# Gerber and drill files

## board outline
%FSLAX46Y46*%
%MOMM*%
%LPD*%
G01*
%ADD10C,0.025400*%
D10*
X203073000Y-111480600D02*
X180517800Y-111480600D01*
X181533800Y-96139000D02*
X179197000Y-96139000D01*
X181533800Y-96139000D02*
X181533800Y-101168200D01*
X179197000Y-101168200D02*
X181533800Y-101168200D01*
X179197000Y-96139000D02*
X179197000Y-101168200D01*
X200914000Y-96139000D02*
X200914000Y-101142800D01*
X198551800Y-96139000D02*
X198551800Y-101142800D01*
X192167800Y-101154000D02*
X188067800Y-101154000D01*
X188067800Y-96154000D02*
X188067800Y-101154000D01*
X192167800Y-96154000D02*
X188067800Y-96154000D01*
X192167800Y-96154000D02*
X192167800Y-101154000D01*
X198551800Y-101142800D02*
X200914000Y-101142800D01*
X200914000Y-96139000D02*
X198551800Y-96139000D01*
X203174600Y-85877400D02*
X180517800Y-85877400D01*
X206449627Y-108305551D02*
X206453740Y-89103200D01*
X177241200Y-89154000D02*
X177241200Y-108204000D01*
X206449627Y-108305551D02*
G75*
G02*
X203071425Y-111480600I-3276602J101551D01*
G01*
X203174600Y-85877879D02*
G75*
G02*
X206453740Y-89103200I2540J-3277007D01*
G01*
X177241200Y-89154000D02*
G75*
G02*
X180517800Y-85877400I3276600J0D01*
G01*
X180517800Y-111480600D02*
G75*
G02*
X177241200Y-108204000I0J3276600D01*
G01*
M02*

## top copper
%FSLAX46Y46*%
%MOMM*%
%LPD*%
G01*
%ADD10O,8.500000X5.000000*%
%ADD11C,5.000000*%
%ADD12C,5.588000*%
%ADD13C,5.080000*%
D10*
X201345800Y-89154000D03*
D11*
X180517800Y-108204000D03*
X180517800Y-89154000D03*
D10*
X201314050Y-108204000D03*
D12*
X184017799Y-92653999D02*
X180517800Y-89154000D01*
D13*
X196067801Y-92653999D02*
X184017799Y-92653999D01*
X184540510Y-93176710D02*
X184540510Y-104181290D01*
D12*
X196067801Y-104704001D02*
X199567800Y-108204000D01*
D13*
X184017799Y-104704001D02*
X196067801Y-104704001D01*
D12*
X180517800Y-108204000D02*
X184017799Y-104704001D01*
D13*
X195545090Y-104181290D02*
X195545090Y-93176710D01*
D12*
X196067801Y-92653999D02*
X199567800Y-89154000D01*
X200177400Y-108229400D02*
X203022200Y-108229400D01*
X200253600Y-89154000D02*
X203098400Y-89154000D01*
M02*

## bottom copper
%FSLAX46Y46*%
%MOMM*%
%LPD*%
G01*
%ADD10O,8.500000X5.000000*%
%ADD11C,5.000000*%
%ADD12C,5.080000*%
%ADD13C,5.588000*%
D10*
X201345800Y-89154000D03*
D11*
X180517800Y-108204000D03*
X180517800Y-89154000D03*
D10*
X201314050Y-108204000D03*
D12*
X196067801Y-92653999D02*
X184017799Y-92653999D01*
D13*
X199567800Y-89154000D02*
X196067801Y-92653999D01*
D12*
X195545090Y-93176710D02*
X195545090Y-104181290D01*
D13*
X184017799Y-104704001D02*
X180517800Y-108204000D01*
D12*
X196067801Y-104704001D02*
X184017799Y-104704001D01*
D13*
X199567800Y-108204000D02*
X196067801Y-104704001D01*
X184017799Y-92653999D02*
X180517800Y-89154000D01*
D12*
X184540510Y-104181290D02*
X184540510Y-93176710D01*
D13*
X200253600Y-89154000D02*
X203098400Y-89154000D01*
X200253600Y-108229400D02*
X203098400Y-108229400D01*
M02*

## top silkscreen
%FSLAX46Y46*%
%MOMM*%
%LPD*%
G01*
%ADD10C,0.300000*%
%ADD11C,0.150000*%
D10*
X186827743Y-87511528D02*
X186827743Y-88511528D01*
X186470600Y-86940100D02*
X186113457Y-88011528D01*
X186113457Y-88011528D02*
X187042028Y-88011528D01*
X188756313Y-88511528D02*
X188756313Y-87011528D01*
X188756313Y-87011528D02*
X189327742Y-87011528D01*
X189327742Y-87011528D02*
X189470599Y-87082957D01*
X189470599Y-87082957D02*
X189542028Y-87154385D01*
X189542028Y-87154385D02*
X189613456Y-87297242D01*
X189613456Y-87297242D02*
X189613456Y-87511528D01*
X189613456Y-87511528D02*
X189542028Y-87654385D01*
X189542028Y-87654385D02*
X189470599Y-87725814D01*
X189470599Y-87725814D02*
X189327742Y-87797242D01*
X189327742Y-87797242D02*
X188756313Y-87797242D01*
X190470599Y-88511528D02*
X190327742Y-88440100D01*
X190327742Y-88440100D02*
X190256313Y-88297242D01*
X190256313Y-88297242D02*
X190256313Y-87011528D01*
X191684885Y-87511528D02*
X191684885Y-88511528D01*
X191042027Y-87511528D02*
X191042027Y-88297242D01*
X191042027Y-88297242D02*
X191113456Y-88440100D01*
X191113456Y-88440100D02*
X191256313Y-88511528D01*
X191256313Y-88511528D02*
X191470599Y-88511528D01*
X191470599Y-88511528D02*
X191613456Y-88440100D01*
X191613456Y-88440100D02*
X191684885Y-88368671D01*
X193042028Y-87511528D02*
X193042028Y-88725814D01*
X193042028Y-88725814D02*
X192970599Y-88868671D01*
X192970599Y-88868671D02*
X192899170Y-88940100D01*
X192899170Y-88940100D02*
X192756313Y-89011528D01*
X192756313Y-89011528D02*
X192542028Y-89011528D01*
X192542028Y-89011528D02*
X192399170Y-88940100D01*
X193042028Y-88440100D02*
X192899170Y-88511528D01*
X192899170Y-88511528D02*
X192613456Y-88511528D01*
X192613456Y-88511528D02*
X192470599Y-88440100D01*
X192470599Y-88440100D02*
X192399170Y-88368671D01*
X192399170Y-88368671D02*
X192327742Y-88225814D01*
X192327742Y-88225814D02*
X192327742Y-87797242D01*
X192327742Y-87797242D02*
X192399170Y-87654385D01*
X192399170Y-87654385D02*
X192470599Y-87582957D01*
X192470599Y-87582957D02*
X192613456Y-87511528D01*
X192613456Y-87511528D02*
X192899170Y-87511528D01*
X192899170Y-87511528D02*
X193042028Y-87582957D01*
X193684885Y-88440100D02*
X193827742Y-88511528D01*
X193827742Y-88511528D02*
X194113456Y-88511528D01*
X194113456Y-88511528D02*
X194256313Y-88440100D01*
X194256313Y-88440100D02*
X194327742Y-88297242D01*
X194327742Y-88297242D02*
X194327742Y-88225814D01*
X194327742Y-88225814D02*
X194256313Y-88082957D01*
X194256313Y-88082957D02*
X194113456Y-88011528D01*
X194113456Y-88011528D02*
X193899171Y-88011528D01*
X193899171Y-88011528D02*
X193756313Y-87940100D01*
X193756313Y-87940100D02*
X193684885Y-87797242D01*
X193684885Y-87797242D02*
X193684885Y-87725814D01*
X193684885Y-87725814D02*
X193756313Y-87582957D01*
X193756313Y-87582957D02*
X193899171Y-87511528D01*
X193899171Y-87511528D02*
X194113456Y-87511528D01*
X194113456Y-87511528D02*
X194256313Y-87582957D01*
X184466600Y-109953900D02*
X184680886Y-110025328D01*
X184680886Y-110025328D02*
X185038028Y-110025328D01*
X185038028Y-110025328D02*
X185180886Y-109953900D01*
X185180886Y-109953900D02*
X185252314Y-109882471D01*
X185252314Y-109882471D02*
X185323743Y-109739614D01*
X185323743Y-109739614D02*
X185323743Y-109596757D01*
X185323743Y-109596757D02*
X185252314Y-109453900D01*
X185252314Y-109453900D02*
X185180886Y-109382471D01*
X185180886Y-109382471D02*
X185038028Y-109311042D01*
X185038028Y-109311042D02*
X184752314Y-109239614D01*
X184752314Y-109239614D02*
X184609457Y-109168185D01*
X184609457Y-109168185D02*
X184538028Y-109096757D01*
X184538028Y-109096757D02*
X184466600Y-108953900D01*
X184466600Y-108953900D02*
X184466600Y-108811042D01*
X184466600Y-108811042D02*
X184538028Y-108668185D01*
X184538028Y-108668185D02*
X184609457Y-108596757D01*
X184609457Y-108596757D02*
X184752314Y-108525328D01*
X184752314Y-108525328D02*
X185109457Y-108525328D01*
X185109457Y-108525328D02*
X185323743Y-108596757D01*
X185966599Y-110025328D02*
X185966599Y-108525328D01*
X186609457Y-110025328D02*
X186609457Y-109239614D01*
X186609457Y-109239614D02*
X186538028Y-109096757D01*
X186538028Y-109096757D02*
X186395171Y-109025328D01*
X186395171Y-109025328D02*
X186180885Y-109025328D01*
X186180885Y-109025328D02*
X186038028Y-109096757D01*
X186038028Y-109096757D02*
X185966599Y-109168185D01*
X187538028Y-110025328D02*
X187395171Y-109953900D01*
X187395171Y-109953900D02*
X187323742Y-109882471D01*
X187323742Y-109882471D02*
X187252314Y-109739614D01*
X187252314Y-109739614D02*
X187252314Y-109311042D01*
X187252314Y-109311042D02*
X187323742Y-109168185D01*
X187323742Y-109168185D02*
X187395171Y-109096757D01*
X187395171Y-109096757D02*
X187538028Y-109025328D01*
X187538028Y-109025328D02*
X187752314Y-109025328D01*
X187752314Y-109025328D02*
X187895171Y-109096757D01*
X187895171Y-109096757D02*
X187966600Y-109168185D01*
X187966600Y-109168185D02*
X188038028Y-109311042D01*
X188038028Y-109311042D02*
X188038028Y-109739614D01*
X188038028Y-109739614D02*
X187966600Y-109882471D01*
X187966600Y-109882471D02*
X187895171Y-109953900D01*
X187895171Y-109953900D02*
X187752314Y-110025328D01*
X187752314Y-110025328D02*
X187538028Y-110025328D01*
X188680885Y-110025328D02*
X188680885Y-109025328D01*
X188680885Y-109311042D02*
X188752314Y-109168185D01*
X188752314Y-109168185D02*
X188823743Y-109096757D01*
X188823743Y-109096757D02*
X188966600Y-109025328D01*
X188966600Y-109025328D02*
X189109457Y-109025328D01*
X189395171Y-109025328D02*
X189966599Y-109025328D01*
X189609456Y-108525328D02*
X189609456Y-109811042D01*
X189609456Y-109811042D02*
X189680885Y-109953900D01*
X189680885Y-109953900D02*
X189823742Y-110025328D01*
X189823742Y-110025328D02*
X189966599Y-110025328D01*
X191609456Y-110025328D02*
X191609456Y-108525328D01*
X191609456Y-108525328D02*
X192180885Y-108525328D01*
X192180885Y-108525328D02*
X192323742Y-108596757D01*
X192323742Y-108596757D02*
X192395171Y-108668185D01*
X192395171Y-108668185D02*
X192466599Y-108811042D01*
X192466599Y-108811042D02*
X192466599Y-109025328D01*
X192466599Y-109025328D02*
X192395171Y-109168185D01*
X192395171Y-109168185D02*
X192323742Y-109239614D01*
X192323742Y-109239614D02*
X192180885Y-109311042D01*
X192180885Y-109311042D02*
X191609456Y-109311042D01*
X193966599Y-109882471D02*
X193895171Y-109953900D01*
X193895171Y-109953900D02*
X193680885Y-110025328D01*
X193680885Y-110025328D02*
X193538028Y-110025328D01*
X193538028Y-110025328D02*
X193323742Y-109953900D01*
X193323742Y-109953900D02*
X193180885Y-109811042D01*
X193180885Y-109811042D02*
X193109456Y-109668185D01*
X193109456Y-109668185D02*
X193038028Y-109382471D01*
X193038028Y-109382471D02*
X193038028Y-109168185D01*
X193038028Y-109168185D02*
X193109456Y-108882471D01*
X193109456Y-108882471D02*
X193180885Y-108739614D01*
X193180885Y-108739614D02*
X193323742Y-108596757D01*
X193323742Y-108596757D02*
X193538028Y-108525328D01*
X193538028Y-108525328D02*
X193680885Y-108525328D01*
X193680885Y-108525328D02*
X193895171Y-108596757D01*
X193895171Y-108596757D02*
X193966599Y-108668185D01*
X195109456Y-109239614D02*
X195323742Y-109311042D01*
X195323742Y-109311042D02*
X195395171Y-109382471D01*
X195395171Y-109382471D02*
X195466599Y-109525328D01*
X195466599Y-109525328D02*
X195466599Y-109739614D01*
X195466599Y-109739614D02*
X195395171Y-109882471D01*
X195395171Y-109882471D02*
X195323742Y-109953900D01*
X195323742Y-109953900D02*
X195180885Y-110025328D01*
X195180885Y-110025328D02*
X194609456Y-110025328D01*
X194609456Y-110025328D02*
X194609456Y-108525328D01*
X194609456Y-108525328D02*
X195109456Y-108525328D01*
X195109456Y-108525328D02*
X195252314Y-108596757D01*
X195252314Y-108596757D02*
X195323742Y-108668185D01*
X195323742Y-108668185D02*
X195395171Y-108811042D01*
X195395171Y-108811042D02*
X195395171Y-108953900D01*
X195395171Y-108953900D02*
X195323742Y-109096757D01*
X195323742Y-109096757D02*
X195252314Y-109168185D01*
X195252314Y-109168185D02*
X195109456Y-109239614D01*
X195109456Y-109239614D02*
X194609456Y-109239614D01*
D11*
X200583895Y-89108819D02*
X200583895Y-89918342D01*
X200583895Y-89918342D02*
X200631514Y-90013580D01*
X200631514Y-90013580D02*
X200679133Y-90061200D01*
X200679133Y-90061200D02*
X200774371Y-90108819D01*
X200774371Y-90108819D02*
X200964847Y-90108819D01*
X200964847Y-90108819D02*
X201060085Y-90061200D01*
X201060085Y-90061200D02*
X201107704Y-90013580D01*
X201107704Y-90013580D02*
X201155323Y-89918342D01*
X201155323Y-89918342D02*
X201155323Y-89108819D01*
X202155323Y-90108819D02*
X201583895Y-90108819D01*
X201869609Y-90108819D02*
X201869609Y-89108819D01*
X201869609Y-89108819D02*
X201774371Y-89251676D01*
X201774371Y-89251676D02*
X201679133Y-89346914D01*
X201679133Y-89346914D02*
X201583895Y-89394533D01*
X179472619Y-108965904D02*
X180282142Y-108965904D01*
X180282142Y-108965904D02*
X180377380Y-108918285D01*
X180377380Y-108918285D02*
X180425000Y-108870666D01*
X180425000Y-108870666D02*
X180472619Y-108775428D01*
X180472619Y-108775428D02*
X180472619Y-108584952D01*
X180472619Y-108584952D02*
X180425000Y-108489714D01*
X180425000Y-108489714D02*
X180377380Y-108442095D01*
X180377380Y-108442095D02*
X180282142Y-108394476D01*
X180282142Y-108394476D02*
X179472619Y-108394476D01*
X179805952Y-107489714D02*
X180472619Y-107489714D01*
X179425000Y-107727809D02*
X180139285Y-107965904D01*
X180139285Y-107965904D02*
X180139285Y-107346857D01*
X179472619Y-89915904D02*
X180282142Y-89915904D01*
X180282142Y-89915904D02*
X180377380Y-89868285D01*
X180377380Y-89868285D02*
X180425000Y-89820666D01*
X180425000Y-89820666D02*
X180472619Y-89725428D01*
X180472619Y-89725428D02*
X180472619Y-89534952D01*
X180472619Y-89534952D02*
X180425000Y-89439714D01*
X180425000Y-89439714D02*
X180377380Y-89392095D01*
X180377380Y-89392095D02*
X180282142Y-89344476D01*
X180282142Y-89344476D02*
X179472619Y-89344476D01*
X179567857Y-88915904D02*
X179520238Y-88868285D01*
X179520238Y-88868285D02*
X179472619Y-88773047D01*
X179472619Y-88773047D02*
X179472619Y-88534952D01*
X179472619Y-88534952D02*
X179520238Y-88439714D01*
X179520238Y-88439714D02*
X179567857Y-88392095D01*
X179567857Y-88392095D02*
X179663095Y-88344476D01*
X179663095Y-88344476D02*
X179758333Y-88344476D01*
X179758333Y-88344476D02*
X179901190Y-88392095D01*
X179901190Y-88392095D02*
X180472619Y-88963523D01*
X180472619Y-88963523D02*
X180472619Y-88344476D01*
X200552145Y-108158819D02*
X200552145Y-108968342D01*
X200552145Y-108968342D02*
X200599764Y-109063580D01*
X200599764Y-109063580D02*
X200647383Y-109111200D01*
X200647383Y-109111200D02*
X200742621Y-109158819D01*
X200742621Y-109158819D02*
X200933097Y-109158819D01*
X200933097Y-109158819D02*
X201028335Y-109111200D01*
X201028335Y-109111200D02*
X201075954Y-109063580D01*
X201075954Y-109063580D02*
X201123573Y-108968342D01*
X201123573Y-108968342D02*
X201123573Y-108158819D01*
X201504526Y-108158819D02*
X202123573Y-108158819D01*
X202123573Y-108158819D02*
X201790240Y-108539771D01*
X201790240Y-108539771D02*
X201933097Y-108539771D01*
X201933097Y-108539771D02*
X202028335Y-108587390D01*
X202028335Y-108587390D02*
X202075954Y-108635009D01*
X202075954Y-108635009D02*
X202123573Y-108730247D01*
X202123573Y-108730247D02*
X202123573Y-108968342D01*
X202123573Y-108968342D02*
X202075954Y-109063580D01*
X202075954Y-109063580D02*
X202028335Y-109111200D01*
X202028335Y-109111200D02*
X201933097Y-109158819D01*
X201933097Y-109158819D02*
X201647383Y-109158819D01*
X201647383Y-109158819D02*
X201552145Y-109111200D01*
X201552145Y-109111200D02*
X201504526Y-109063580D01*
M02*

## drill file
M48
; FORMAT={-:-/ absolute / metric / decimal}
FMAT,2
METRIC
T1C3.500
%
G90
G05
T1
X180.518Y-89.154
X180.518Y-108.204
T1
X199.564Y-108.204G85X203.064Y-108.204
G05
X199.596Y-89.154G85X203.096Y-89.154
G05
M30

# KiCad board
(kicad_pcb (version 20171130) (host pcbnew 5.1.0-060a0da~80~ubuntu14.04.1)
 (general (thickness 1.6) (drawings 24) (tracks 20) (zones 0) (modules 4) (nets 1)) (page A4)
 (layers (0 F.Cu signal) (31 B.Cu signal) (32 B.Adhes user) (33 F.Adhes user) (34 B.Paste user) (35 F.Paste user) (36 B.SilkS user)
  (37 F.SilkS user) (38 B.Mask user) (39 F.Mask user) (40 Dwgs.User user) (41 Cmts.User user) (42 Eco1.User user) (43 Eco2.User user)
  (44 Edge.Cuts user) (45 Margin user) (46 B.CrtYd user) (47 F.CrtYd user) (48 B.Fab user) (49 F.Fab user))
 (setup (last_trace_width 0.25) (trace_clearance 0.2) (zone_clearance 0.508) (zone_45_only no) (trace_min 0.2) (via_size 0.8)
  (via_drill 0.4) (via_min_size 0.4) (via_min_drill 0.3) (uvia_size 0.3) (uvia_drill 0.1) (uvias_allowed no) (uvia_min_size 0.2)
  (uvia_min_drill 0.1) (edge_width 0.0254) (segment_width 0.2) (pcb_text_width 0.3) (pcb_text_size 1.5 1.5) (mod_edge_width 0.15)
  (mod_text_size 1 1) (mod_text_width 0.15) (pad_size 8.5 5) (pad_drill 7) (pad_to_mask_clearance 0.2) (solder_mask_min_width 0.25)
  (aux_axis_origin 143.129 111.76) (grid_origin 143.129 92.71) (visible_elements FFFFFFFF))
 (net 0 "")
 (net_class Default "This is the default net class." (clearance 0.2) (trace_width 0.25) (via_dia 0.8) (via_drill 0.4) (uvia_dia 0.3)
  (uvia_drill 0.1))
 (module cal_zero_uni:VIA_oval (layer F.Cu) (at 201.3458 89.154)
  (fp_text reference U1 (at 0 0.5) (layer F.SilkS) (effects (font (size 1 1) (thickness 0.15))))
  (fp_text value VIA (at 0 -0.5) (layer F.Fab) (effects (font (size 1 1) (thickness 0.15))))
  (pad 1 thru_hole oval (at 0 0) (size 8.5 5) (drill oval 7 3.5) (layers *.Cu *.Mask)))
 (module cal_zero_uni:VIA (layer F.Cu) (at 180.5178 108.204 270)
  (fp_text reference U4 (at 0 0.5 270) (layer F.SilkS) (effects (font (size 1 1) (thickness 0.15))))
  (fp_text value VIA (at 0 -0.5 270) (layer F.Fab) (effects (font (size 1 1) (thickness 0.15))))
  (pad 1 thru_hole circle (at 0 0 270) (size 5 5) (drill 3.5) (layers *.Cu *.Mask)))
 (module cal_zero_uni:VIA (layer F.Cu) (at 180.5178 89.154 270)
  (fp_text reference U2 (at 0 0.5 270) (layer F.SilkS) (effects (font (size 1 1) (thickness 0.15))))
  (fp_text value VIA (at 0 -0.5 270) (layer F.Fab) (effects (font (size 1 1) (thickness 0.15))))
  (pad 1 thru_hole circle (at 0 0 270) (size 5 5) (drill 3.5) (layers *.Cu *.Mask)))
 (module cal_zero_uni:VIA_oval (layer F.Cu) (at 201.31405 108.204)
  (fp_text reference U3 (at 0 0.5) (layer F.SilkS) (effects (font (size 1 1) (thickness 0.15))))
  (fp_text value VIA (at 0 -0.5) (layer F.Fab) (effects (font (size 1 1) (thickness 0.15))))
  (pad 1 thru_hole oval (at 0 0) (size 8.5 5) (drill oval 7 3.5) (layers *.Cu *.Mask)))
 (gr_line (start 203.073 111.4806) (end 180.5178 111.4806) (layer Edge.Cuts) (width 0.0254))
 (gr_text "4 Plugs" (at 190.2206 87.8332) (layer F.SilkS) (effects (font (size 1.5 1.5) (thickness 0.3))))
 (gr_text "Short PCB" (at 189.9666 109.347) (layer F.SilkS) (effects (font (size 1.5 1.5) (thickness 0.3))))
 (gr_line (start 181.5338 96.139) (end 179.197 96.139) (layer Edge.Cuts) (width 0.0254))
 (gr_line (start 181.5338 96.139) (end 181.5338 101.1682) (layer Edge.Cuts) (width 0.0254))
 (gr_line (start 179.197 101.1682) (end 181.5338 101.1682) (layer Edge.Cuts) (width 0.0254))
 (gr_line (start 179.197 96.139) (end 179.197 101.1682) (layer Edge.Cuts) (width 0.0254))
 (gr_line (start 200.914 96.139) (end 200.914 101.1428) (layer Edge.Cuts) (width 0.0254))
 (gr_line (start 198.5518 96.139) (end 198.5518 101.1428) (layer Edge.Cuts) (width 0.0254))
 (gr_line (start 192.1678 101.154) (end 188.0678 101.154) (layer Edge.Cuts) (width 0.0254))
 (gr_line (start 188.0678 96.154) (end 188.0678 101.154) (layer Edge.Cuts) (width 0.0254))
 (gr_line (start 192.1678 96.154) (end 188.0678 96.154) (layer Edge.Cuts) (width 0.0254))
 (gr_line (start 192.1678 96.154) (end 192.1678 101.154) (layer Edge.Cuts) (width 0.0254))
 (gr_line (start 198.5518 101.1428) (end 200.914 101.1428) (layer Edge.Cuts) (width 0.0254))
 (gr_line (start 200.914 96.139) (end 198.5518 96.139) (layer Edge.Cuts) (width 0.0254))
 (gr_line (start 203.1746 85.8774) (end 180.5178 85.8774) (layer Edge.Cuts) (width 0.0254))
 (gr_line (start 206.449627 108.305551) (end 206.45374 89.1032) (layer Edge.Cuts) (width 0.0254))
 (gr_line (start 177.2412 89.154) (end 177.2412 108.204) (layer Edge.Cuts) (width 0.0254))
 (gr_arc (start 203.173025 108.204) (end 203.071425 111.4806) (angle -90.00085275) (layer Edge.Cuts) (width 0.0254))
 (gr_arc (start 203.17714 89.154886) (end 206.45374 89.1032) (angle -89.14068518) (layer Edge.Cuts) (width 0.0254))
 (gr_arc (start 180.5178 89.154) (end 180.5178 85.8774) (angle -90) (layer Edge.Cuts) (width 0.0254))
 (gr_arc (start 180.5178 108.204) (end 177.2412 108.204) (angle -90) (layer Edge.Cuts) (width 0.0254))
 (segment (start 184.017799 92.653999) (end 180.5178 89.154) (width 5.588) (layer F.Cu) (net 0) (status 20))
 (segment (start 196.067801 92.653999) (end 184.017799 92.653999) (width 5.08) (layer F.Cu) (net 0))
 (segment (start 184.54051 93.17671) (end 184.54051 104.18129) (width 5.08) (layer F.Cu) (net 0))
 (segment (start 196.067801 104.704001) (end 199.5678 108.204) (width 5.588) (layer F.Cu) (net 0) (status 20))
 (segment (start 184.017799 104.704001) (end 196.067801 104.704001) (width 5.08) (layer F.Cu) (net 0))
 (segment (start 180.5178 108.204) (end 184.017799 104.704001) (width 5.588) (layer F.Cu) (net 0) (status 10))
 (segment (start 195.54509 104.18129) (end 195.54509 93.17671) (width 5.08) (layer F.Cu) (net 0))
 (segment (start 196.067801 92.653999) (end 199.5678 89.154) (width 5.588) (layer F.Cu) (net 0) (status 20))
 (segment (start 196.067801 92.653999) (end 184.017799 92.653999) (width 5.08) (layer B.Cu) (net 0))
 (segment (start 199.5678 89.154) (end 196.067801 92.653999) (width 5.588) (layer B.Cu) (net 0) (status 10))
 (segment (start 195.54509 93.17671) (end 195.54509 104.18129) (width 5.08) (layer B.Cu) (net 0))
 (segment (start 184.017799 104.704001) (end 180.5178 108.204) (width 5.588) (layer B.Cu) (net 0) (status 20))
 (segment (start 196.067801 104.704001) (end 184.017799 104.704001) (width 5.08) (layer B.Cu) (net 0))
 (segment (start 199.5678 108.204) (end 196.067801 104.704001) (width 5.588) (layer B.Cu) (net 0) (status 10))
 (segment (start 184.017799 92.653999) (end 180.5178 89.154) (width 5.588) (layer B.Cu) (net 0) (status 20))
 (segment (start 184.54051 104.18129) (end 184.54051 93.17671) (width 5.08) (layer B.Cu) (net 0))
 (segment (start 200.2536 89.154) (end 203.0984 89.154) (width 5.588) (layer B.Cu) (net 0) (status 30))
 (segment (start 200.1774 108.2294) (end 203.0222 108.2294) (width 5.588) (layer F.Cu) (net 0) (status 30))
 (segment (start 200.2536 89.154) (end 203.0984 89.154) (width 5.588) (layer F.Cu) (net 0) (status 30))
 (segment (start 200.2536 108.2294) (end 203.0984 108.2294) (width 5.588) (layer B.Cu) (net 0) (status 30)))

